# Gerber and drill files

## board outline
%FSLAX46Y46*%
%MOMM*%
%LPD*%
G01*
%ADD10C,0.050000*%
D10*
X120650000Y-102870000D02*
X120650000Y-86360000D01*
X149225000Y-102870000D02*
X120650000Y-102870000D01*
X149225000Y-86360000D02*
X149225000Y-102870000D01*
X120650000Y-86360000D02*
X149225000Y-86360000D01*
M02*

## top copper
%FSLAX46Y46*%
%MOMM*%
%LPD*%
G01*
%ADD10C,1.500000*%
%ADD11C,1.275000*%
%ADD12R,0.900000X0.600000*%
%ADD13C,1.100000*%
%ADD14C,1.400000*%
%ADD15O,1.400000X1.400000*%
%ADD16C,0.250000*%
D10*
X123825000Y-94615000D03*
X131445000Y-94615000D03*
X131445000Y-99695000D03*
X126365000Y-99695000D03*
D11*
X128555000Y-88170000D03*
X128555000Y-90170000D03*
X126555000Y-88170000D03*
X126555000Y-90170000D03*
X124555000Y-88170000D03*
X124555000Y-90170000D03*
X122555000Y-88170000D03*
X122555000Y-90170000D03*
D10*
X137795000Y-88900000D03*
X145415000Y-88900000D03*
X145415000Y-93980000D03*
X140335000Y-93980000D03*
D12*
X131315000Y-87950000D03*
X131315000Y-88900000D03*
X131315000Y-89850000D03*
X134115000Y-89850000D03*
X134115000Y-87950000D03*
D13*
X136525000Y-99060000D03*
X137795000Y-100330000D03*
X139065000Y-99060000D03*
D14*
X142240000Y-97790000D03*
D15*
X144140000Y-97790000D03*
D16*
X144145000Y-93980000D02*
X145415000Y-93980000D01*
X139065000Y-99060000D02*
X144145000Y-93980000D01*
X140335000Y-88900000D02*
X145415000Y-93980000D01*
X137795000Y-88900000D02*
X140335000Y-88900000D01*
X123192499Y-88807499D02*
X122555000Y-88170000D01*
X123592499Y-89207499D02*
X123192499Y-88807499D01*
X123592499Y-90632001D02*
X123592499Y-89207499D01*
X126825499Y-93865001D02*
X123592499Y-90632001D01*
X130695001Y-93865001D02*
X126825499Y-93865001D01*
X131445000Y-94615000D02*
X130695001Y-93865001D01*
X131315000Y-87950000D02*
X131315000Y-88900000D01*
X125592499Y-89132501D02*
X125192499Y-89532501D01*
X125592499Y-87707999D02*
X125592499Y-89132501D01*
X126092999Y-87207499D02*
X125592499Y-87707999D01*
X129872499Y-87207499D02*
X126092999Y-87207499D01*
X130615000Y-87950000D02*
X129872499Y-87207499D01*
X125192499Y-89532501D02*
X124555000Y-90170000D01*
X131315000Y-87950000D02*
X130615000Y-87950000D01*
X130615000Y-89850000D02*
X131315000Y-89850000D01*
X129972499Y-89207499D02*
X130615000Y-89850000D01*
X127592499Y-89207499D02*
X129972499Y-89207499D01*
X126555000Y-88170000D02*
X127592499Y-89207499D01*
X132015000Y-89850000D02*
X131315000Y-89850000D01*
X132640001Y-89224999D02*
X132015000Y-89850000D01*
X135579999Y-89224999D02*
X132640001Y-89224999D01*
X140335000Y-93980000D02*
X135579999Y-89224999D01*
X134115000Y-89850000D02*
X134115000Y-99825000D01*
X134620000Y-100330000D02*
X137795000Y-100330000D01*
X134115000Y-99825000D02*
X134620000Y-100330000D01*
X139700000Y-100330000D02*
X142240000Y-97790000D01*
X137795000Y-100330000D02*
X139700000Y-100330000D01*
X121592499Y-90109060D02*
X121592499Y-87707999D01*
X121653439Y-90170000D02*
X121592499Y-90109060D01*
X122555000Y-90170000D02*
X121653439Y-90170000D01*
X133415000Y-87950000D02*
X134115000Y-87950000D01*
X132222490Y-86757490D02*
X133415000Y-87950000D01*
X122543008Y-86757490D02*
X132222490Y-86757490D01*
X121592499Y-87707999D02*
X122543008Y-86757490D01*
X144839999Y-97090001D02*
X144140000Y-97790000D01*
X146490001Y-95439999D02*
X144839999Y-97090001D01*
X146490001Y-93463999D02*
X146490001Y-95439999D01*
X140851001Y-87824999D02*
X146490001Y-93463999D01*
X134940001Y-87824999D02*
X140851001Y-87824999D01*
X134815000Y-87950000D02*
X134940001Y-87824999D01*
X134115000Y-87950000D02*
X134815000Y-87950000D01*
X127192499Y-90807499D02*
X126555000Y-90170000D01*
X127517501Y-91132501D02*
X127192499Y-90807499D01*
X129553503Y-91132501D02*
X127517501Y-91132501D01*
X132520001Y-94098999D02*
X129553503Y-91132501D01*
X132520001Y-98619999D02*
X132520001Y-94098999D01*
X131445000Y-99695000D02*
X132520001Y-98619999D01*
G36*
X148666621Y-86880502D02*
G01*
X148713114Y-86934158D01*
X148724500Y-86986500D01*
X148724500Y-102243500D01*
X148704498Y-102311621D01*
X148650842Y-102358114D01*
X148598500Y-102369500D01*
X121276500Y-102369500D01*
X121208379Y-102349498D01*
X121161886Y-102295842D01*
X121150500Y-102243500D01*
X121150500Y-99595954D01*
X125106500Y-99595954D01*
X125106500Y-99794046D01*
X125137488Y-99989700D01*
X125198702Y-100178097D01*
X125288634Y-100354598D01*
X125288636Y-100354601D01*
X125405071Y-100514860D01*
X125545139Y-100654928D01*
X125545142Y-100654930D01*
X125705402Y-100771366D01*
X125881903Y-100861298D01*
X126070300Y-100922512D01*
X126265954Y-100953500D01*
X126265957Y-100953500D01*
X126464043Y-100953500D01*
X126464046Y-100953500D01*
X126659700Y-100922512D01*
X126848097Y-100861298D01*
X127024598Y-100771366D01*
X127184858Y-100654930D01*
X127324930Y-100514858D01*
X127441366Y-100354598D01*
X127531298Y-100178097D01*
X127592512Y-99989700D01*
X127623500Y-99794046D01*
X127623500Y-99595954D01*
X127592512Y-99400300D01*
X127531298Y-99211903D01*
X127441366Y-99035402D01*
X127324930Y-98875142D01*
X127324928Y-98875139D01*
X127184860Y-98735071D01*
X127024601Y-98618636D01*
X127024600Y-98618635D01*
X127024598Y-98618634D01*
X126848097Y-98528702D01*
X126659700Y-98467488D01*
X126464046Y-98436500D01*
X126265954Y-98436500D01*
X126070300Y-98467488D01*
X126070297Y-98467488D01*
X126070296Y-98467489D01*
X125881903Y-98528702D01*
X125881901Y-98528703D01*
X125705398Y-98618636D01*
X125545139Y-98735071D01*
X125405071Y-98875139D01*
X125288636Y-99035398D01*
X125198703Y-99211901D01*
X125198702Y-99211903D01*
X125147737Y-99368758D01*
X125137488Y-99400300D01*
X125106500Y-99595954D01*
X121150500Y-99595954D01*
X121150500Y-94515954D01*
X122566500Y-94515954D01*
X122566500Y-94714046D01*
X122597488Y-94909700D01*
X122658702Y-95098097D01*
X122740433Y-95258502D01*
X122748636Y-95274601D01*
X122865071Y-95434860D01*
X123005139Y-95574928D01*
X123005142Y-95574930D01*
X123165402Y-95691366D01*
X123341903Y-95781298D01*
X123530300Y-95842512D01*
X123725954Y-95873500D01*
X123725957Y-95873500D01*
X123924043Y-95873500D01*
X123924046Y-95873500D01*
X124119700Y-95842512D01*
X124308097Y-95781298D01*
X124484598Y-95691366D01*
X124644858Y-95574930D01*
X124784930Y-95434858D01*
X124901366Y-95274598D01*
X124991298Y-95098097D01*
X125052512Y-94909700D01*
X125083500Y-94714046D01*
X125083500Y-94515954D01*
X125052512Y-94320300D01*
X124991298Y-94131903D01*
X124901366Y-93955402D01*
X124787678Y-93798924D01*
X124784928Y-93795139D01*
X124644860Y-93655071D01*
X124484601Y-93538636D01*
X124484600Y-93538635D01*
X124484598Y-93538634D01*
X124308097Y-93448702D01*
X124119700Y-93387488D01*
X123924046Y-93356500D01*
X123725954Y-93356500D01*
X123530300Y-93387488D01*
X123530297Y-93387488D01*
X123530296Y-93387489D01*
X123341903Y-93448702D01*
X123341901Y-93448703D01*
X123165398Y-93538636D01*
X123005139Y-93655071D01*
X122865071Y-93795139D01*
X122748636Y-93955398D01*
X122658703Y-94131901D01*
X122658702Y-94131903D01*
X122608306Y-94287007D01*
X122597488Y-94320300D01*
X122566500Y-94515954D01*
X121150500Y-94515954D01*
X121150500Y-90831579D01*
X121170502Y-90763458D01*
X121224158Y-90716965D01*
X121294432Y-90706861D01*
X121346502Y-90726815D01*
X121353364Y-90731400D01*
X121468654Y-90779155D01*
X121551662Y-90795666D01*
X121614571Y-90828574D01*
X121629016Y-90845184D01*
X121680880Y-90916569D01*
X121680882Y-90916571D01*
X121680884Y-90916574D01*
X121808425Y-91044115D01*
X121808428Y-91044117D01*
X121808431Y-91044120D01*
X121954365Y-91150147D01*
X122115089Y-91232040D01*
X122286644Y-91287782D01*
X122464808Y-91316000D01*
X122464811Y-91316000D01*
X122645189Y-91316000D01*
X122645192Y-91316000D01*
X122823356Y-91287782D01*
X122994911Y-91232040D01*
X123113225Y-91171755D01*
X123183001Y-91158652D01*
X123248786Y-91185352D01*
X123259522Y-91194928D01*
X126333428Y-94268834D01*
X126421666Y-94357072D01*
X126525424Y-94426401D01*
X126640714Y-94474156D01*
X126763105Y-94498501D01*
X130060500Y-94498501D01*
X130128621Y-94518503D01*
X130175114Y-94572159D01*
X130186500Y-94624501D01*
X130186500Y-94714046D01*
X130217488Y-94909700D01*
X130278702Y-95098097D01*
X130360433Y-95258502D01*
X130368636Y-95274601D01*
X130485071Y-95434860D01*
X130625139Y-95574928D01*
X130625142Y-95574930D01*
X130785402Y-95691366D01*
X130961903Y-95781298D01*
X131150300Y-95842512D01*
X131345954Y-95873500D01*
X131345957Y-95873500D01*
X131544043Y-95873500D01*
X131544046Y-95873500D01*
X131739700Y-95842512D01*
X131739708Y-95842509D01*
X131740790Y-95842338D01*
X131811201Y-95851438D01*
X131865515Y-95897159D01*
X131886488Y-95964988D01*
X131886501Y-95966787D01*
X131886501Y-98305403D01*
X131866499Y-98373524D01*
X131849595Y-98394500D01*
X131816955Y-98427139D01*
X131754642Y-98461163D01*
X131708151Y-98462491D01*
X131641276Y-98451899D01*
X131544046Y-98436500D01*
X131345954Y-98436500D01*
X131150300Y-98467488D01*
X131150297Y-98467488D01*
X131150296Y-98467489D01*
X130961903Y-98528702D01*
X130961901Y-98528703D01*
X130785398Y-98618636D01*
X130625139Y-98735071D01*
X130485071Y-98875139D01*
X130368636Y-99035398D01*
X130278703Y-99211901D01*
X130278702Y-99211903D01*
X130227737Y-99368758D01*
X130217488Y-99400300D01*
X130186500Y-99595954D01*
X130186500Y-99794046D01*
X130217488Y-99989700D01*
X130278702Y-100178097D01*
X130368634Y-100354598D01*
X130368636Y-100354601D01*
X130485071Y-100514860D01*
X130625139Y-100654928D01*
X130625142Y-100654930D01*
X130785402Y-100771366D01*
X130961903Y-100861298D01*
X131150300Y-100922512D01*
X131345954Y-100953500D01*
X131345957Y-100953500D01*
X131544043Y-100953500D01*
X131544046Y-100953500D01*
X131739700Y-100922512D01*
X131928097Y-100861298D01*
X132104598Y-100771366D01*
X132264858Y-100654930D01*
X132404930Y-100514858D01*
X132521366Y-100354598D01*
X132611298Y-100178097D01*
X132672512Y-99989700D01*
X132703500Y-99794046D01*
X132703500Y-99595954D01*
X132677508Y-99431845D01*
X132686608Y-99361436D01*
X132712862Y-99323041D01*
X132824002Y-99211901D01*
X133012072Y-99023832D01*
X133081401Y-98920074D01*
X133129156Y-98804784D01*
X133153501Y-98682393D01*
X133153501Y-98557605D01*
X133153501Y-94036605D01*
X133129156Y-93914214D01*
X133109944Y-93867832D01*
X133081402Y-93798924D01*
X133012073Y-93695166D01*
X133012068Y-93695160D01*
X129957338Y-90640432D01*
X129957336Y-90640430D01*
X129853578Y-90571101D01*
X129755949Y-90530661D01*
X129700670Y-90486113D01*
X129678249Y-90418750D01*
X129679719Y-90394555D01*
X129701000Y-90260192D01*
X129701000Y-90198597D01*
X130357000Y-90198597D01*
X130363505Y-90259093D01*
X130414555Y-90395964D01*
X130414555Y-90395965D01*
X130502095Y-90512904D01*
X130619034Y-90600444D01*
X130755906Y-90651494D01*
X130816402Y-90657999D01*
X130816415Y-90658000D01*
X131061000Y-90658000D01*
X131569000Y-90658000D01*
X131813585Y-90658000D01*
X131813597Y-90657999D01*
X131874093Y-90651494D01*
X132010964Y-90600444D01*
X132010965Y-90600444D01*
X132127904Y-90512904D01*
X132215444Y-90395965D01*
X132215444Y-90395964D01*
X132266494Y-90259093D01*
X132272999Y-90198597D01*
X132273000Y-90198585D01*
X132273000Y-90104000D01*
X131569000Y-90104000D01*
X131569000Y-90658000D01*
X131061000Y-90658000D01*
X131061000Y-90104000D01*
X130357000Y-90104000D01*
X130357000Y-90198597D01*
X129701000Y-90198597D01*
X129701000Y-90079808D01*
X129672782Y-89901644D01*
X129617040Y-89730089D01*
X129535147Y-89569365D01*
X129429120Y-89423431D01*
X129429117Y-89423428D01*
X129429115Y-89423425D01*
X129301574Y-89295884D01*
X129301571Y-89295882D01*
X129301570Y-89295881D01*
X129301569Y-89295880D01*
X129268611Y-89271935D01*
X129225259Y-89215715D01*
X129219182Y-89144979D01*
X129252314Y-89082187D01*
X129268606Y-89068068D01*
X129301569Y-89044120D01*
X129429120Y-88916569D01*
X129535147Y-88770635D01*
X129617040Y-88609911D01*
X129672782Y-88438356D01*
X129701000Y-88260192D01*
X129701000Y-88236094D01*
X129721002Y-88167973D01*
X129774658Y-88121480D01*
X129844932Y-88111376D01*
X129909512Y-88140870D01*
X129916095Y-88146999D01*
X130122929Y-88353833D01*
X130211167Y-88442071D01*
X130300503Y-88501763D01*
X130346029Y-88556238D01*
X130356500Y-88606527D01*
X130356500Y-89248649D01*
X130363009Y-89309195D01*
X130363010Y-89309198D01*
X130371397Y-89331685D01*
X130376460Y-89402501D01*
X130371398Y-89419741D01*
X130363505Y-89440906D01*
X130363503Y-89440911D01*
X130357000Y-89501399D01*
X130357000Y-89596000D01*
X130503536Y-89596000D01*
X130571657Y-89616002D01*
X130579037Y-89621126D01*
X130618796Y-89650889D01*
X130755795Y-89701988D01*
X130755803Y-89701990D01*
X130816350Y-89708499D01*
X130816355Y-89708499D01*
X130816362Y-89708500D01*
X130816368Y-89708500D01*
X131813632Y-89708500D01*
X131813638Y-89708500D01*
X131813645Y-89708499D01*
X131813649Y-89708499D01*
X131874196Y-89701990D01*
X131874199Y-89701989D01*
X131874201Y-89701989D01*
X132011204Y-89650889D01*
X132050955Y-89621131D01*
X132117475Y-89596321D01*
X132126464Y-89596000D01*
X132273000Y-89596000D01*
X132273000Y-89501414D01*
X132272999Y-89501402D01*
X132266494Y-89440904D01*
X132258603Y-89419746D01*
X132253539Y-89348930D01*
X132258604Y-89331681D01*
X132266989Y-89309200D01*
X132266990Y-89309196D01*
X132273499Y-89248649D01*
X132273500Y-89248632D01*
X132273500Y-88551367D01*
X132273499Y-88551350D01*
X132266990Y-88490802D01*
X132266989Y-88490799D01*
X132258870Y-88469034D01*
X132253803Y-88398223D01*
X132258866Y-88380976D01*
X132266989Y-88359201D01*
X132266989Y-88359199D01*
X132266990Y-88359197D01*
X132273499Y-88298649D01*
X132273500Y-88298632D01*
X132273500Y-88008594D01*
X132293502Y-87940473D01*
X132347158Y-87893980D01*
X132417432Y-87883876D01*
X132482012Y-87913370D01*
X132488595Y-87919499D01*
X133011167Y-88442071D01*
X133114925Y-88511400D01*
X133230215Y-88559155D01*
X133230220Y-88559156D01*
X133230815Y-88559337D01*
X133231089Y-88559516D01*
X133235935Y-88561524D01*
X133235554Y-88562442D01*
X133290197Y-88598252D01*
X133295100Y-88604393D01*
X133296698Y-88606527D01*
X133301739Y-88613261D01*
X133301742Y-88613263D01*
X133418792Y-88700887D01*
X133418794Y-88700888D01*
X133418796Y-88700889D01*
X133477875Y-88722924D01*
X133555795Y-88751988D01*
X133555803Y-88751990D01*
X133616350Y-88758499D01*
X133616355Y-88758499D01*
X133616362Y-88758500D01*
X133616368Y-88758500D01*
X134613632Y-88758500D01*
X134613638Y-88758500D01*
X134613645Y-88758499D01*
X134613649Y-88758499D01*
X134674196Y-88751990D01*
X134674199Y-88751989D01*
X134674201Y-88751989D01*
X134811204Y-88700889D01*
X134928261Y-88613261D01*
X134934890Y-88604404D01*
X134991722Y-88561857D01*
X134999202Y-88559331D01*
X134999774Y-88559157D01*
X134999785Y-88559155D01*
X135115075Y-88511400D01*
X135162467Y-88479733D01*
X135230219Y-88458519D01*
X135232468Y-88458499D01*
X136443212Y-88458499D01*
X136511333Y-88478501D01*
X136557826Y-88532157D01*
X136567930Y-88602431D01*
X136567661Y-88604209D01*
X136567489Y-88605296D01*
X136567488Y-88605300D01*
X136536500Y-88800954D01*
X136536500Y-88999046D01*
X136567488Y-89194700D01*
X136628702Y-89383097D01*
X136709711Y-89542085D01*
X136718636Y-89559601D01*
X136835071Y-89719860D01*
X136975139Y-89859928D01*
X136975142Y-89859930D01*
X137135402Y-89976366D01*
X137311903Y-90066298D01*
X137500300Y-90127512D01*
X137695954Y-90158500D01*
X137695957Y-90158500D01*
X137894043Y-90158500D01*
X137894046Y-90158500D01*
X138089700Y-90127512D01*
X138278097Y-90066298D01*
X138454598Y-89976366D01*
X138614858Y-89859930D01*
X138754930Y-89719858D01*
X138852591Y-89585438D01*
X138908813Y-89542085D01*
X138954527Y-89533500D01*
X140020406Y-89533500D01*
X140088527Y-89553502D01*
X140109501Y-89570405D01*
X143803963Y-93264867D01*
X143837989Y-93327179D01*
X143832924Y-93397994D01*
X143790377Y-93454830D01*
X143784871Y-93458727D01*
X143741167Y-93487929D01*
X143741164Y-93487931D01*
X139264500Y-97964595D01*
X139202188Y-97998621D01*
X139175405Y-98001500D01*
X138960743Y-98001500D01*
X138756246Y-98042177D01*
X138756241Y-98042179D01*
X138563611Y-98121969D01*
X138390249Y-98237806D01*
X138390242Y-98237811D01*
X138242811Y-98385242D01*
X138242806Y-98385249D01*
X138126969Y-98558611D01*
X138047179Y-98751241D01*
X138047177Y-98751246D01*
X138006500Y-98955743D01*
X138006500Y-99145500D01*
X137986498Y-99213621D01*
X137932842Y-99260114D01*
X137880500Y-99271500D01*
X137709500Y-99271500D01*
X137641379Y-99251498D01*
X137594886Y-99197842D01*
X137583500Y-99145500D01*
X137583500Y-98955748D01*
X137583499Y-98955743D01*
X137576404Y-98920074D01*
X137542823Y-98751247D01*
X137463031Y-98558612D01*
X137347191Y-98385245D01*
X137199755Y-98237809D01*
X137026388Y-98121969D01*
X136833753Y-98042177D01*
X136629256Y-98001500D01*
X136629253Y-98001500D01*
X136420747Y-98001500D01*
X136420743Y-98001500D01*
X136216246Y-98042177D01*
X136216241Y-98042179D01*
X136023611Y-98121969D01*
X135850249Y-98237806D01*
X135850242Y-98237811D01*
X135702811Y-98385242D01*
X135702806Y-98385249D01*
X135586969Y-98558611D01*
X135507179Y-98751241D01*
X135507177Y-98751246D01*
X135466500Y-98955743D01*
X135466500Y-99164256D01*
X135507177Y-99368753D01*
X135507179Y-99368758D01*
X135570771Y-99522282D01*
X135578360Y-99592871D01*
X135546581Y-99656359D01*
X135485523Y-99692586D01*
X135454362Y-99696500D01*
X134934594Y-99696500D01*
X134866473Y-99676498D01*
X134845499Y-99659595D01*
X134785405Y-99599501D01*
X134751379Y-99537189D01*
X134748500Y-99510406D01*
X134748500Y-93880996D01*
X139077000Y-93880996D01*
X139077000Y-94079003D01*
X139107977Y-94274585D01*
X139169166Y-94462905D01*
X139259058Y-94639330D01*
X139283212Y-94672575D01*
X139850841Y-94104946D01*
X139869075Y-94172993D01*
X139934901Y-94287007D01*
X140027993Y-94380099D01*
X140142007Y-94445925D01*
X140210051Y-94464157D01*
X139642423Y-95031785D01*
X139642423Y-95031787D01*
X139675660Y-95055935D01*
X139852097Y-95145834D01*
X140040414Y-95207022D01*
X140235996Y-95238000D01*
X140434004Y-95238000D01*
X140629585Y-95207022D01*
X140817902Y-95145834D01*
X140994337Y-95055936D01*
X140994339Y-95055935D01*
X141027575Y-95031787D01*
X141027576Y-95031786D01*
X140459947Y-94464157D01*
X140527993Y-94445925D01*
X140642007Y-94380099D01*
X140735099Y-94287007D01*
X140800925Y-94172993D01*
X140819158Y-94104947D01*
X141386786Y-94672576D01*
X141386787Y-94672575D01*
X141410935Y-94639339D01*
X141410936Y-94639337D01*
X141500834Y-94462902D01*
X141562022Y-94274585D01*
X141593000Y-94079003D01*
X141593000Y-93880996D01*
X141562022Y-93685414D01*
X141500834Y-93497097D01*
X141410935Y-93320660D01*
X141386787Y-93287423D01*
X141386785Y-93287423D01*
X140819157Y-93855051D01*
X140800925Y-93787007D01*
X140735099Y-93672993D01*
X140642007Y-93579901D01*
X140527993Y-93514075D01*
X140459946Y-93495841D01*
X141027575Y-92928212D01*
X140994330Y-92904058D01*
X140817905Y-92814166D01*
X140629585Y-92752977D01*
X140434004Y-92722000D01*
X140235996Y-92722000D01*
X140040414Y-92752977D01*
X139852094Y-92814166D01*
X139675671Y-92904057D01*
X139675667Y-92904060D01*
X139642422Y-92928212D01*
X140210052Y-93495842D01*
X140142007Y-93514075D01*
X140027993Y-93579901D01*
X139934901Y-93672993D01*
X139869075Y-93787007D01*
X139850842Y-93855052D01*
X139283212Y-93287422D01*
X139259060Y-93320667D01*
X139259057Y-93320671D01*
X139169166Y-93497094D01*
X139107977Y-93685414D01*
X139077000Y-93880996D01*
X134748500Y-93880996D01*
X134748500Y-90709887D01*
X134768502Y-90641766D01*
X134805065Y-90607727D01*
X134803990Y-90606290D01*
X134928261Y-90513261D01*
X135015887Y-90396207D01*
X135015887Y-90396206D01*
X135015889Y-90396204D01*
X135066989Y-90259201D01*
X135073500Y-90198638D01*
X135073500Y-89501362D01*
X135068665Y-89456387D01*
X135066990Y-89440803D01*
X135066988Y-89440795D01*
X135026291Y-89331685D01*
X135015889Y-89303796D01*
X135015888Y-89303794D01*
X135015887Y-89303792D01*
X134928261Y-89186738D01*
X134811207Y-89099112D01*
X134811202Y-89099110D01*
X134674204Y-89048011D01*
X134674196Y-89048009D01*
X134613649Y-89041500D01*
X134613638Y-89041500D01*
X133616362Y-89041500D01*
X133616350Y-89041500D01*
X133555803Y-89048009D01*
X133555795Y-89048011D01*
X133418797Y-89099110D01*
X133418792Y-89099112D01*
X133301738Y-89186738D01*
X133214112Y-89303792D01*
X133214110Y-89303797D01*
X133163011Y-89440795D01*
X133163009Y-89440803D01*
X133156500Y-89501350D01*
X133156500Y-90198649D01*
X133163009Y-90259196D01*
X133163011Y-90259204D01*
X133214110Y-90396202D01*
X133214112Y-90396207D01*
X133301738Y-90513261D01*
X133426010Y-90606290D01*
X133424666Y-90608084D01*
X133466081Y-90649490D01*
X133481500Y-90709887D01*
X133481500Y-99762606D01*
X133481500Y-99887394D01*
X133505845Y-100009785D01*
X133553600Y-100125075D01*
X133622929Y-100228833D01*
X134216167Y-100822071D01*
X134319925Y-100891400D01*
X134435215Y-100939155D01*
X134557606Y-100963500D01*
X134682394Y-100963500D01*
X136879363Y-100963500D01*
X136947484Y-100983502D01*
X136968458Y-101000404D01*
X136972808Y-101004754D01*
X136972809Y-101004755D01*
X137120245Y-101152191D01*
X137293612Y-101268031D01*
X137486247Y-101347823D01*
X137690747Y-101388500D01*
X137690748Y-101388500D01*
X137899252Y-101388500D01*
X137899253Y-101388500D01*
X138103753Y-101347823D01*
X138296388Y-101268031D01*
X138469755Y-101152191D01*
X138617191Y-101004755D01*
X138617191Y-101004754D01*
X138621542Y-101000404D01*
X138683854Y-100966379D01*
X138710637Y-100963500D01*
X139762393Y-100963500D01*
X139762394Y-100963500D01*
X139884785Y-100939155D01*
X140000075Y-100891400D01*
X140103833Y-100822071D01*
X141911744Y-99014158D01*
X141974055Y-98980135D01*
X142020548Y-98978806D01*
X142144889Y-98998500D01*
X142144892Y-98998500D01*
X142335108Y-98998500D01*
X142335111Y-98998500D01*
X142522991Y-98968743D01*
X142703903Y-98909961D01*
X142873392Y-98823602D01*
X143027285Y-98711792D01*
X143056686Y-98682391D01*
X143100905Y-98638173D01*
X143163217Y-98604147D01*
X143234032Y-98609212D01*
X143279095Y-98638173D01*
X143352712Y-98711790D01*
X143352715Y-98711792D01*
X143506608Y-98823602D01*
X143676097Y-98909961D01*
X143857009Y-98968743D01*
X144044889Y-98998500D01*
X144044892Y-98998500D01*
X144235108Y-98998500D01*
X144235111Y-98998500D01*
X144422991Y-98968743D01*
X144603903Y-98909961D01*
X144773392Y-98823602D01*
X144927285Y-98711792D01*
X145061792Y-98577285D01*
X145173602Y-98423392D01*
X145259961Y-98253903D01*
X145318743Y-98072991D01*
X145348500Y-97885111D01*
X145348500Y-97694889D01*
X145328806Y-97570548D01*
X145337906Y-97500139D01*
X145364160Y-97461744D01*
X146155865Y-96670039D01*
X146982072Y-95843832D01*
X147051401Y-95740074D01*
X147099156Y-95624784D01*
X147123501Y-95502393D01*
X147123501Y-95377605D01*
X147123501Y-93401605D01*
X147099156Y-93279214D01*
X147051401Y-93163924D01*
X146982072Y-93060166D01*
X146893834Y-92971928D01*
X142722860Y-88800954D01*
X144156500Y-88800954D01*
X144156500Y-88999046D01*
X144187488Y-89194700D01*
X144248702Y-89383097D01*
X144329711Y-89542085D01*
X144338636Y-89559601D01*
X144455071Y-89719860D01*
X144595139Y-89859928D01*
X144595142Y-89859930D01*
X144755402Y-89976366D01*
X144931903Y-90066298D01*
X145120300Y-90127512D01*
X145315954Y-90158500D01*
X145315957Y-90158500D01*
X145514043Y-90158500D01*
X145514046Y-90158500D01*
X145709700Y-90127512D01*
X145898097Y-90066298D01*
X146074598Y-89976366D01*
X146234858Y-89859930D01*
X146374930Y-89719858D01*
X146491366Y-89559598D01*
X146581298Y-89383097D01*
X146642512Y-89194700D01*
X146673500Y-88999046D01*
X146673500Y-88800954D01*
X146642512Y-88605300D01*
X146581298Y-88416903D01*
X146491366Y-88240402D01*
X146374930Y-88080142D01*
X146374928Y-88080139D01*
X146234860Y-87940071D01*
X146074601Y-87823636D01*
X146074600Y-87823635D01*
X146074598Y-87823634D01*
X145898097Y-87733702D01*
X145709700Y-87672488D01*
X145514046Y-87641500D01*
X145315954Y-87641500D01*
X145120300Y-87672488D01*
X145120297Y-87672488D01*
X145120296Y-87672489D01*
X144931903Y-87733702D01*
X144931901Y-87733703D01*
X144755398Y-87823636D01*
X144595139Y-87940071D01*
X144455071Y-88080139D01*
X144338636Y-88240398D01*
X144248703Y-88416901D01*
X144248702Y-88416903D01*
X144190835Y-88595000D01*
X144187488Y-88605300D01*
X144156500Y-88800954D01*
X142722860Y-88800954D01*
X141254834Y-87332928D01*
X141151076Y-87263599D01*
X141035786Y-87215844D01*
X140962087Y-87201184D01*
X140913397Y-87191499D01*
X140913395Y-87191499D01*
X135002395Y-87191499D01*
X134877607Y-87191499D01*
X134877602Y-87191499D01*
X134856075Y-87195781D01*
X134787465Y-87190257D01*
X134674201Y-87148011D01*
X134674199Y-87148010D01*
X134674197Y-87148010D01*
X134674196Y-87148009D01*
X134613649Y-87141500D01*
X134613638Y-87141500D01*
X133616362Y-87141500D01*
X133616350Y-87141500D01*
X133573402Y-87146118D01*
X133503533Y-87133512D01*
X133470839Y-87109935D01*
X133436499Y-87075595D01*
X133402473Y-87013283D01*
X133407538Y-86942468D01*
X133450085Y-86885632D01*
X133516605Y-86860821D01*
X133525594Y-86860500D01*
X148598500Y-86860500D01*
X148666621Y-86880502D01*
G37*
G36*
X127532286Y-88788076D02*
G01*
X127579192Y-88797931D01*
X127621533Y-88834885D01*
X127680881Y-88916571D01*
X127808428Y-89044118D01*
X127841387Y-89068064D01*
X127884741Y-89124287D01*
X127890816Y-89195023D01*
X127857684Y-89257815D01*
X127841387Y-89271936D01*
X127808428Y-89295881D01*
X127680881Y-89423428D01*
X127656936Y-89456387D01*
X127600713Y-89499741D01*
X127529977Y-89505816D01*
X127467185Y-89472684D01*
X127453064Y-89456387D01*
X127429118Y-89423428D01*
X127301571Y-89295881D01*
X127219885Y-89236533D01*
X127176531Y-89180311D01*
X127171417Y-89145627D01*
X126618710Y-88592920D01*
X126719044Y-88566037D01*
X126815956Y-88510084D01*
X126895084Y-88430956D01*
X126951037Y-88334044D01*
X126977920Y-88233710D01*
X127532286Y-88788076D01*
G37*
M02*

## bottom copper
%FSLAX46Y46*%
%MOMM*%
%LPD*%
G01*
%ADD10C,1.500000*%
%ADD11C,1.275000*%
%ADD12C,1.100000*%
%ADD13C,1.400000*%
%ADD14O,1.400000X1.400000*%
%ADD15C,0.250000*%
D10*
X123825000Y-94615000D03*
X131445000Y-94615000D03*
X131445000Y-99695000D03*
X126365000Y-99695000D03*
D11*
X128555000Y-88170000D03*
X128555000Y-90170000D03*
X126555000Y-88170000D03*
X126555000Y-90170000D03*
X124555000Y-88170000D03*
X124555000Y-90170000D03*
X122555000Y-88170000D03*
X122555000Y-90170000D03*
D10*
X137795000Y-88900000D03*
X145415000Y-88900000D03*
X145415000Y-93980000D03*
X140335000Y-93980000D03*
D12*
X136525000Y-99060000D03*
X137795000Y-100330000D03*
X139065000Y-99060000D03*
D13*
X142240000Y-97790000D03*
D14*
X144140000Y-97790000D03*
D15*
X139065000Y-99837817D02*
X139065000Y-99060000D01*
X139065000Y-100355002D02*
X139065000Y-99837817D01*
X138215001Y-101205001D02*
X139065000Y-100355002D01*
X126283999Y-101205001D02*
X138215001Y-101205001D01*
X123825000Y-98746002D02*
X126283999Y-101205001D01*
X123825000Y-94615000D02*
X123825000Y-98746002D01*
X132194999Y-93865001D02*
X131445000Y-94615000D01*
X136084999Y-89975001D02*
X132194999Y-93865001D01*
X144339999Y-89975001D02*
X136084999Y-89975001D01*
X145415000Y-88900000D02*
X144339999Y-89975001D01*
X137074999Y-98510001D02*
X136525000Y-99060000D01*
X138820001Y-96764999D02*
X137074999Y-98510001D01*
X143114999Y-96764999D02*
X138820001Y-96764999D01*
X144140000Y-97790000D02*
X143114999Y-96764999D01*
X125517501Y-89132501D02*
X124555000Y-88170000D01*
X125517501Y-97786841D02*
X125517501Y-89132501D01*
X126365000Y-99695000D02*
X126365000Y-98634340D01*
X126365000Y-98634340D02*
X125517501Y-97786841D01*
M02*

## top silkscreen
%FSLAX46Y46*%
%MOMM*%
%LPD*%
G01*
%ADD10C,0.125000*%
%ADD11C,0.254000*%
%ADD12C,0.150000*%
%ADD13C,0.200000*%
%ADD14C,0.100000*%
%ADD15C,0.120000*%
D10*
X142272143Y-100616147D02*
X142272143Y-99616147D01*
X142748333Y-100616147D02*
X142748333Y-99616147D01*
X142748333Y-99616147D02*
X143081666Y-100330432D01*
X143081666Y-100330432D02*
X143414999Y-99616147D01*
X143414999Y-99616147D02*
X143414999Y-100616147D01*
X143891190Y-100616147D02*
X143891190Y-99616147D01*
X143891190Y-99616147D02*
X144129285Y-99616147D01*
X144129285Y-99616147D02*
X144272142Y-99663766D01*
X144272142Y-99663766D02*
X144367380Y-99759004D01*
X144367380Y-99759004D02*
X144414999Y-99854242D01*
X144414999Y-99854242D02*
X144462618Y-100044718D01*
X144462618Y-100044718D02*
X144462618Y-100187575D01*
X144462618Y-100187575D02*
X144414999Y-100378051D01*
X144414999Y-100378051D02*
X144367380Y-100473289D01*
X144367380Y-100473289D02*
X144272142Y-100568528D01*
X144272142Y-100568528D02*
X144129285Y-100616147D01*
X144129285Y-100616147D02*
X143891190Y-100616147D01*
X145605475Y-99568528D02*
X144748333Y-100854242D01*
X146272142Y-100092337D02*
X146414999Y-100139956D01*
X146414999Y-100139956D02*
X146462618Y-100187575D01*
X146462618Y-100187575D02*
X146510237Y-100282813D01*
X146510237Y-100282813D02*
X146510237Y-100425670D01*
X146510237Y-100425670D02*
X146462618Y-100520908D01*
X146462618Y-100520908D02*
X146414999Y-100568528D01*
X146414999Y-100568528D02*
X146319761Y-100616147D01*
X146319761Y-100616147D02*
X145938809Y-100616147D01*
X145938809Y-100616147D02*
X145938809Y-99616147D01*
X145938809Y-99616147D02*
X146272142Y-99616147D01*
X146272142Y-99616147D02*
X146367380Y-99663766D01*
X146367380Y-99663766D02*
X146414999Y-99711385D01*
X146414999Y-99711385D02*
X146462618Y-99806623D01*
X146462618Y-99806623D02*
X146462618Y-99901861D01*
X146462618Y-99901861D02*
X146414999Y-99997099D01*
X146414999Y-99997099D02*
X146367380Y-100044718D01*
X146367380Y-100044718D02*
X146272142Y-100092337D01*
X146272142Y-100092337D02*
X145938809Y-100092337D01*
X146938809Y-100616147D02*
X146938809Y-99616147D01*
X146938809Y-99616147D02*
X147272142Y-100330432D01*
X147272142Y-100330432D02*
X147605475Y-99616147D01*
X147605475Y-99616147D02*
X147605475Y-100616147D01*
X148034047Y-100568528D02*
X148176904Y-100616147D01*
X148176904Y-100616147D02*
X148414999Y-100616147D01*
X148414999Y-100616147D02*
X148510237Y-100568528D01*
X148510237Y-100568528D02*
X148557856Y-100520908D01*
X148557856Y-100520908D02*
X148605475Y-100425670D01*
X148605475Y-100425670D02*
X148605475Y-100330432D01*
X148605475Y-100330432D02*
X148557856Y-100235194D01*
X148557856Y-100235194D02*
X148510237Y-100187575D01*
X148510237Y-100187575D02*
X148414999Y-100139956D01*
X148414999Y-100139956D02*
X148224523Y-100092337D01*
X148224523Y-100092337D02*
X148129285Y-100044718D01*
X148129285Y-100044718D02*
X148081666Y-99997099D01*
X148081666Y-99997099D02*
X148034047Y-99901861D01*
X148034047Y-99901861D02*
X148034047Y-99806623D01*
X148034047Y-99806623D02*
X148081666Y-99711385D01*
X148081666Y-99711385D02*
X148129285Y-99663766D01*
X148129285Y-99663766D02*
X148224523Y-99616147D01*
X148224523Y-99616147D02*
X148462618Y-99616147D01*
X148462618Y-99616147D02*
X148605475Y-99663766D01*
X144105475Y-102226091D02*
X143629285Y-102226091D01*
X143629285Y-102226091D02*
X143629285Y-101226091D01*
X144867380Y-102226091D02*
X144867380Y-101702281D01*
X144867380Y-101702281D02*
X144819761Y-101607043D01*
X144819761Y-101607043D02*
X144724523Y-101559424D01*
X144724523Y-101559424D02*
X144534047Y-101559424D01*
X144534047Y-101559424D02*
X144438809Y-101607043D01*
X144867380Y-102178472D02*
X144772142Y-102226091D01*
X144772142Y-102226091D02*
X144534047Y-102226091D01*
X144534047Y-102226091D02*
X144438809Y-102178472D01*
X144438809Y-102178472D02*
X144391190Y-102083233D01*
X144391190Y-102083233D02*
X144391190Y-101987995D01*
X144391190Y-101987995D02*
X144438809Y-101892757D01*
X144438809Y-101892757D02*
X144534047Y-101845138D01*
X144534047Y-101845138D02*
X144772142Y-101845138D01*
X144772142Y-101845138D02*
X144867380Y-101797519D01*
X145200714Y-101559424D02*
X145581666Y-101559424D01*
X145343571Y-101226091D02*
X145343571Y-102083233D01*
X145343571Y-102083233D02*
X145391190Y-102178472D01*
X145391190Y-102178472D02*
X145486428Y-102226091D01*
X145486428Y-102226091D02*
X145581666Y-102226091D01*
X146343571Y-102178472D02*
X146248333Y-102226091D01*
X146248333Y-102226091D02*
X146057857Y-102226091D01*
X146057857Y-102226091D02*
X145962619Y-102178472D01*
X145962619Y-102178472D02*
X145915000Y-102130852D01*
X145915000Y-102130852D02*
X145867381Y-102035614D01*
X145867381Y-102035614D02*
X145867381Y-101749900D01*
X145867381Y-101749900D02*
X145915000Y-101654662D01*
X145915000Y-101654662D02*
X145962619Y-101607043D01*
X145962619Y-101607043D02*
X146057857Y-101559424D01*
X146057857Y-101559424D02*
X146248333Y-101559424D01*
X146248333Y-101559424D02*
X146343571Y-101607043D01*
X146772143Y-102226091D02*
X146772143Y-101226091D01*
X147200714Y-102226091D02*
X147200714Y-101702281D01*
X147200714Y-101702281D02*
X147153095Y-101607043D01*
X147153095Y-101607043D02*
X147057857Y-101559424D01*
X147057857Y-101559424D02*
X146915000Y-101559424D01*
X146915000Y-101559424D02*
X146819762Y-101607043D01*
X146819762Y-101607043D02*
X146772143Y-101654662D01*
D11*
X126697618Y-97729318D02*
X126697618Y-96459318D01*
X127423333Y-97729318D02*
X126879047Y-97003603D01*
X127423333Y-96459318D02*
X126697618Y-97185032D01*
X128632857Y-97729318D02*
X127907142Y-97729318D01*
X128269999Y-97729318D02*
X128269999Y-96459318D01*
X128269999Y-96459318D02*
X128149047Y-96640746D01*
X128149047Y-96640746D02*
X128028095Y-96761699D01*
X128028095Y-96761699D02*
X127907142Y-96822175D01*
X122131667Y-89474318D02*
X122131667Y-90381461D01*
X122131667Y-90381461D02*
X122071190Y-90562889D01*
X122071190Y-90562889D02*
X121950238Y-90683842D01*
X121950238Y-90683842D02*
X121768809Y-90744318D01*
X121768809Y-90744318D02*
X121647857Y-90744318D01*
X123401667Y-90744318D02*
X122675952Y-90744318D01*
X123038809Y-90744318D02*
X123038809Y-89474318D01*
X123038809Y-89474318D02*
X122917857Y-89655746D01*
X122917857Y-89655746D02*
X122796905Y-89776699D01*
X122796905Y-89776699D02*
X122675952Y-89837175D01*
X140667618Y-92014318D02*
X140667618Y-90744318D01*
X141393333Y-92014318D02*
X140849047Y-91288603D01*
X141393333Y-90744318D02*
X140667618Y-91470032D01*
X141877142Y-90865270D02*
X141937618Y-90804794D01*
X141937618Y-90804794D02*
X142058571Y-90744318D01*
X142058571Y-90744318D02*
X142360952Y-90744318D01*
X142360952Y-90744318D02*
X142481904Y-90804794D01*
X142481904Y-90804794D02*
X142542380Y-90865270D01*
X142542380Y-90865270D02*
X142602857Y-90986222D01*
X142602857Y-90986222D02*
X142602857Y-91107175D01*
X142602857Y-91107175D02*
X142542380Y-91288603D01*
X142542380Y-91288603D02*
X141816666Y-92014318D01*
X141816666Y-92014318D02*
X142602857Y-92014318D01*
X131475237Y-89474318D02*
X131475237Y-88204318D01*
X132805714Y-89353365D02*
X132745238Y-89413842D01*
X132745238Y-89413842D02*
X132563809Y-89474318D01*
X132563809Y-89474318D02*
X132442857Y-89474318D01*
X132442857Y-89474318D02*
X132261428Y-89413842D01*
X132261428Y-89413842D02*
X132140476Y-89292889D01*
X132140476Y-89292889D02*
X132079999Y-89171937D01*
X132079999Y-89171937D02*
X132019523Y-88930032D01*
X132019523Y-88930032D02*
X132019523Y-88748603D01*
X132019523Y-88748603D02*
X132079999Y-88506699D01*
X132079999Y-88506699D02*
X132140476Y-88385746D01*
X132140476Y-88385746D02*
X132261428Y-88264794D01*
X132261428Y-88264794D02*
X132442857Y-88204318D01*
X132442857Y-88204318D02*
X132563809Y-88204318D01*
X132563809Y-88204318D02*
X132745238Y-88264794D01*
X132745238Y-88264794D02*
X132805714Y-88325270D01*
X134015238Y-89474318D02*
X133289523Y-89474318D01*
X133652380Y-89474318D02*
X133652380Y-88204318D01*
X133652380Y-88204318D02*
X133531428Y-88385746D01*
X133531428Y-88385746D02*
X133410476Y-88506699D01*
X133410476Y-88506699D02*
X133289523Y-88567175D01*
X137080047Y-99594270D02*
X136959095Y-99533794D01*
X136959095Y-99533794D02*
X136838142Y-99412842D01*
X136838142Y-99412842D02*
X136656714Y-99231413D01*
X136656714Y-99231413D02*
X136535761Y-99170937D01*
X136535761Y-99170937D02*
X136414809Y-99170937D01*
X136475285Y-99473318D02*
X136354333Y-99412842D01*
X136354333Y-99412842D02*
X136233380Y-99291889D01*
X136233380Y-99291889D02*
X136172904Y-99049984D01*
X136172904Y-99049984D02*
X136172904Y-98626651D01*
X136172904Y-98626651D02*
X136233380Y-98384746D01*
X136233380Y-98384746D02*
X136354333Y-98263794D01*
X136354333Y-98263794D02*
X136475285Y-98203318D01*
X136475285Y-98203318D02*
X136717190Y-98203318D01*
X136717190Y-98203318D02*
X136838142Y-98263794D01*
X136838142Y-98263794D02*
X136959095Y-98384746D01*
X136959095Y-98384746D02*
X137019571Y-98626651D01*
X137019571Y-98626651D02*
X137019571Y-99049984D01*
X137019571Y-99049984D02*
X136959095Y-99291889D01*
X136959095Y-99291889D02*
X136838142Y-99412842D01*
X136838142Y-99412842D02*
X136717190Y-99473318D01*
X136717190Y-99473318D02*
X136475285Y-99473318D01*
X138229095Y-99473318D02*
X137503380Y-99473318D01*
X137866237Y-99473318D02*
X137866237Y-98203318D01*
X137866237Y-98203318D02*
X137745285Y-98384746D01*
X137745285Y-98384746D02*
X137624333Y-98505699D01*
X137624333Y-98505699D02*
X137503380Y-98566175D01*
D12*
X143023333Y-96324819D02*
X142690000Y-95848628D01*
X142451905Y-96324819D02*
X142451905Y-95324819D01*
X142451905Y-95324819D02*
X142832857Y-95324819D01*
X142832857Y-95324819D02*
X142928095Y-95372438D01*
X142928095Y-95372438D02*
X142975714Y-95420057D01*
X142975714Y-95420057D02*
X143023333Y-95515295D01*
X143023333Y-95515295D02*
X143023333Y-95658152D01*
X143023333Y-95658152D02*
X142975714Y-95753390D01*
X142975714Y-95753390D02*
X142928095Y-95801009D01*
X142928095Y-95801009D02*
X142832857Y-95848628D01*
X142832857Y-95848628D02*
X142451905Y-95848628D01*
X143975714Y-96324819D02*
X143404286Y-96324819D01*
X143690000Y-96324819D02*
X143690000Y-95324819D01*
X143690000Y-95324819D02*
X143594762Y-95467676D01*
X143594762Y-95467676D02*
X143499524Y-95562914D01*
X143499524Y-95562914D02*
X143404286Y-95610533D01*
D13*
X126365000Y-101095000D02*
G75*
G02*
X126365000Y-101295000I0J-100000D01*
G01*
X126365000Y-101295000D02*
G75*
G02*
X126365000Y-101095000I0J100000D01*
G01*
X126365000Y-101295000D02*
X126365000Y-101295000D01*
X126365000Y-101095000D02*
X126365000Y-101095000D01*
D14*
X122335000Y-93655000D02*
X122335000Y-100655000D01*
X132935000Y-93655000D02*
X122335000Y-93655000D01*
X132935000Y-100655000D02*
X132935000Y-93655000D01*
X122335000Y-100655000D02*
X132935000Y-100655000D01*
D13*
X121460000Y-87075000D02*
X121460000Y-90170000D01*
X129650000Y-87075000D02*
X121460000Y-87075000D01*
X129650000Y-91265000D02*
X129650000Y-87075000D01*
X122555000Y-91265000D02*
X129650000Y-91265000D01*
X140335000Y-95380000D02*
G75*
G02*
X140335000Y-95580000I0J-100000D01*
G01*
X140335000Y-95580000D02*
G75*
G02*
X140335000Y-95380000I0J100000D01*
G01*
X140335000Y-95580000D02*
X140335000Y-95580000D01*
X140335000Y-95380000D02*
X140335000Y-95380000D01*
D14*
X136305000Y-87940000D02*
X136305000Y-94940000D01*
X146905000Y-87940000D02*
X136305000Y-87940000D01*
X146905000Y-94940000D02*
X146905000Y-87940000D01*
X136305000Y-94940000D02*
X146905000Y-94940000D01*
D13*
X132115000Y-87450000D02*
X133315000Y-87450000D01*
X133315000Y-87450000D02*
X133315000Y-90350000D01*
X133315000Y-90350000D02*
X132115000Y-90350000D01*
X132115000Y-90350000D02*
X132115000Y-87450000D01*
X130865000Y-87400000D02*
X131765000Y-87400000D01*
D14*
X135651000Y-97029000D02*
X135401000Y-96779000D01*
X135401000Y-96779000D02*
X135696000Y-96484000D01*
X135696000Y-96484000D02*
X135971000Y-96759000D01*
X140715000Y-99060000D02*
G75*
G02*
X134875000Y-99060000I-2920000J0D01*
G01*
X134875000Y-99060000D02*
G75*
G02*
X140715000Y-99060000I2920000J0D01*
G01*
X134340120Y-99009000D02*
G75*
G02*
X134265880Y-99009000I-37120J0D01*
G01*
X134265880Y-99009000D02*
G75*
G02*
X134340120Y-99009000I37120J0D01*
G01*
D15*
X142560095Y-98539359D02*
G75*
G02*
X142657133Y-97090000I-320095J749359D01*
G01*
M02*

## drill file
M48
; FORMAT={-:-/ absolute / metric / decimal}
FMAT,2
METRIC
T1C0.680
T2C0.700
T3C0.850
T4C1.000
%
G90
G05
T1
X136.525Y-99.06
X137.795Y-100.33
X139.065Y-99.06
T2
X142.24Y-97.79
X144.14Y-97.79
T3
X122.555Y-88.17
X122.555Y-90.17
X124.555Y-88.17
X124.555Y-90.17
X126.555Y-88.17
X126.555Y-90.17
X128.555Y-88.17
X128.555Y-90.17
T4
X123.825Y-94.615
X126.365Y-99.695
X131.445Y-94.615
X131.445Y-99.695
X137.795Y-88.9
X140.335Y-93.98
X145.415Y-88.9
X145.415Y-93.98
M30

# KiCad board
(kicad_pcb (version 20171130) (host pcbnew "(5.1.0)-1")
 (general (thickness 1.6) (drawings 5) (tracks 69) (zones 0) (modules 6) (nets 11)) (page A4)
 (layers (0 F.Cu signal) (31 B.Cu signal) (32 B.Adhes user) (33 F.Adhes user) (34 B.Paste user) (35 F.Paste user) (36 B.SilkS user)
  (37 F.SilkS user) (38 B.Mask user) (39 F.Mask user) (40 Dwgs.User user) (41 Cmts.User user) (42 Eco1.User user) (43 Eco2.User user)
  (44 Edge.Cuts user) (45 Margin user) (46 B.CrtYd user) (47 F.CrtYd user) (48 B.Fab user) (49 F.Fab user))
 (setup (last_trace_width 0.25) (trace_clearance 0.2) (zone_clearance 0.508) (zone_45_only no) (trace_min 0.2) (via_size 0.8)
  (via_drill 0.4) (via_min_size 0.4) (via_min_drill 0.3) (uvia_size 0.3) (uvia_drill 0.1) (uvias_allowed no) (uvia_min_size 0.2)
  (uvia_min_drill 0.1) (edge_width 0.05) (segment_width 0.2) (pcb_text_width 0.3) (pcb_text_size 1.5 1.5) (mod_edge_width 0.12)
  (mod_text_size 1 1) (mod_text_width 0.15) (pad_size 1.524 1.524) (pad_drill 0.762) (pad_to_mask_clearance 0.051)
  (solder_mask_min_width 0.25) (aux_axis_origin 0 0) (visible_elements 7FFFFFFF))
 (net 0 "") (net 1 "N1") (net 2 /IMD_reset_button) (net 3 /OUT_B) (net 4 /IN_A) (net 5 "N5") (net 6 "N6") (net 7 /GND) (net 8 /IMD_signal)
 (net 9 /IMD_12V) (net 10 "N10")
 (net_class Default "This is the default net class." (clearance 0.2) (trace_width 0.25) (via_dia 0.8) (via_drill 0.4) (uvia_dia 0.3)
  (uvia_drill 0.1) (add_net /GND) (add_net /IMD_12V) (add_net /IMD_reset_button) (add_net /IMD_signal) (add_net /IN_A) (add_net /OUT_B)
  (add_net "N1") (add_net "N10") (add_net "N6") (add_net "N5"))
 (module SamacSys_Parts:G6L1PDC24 (layer F.Cu) (at 126.365 99.695)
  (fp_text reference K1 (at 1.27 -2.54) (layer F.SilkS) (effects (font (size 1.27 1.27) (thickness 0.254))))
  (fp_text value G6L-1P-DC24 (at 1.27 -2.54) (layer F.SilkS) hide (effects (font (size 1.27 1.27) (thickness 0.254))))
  (fp_arc (start 0 1.5) (end 0 1.6) (angle -180) (layer F.SilkS) (width 0.2))
  (fp_arc (start 0 1.5) (end 0 1.4) (angle -180) (layer F.SilkS) (width 0.2))
  (fp_line (start 0 1.6) (end 0 1.6) (layer F.SilkS) (width 0.2))
  (fp_line (start 0 1.4) (end 0 1.4) (layer F.SilkS) (width 0.2))
  (fp_line (start -4.03 -6.04) (end -4.03 0.96) (layer F.SilkS) (width 0.1))
  (fp_line (start 6.57 -6.04) (end -4.03 -6.04) (layer F.SilkS) (width 0.1))
  (fp_line (start 6.57 0.96) (end 6.57 -6.04) (layer F.SilkS) (width 0.1))
  (fp_line (start -4.03 0.96) (end 6.57 0.96) (layer F.SilkS) (width 0.1))
  (pad 8 thru_hole circle (at -2.54 -5.08) (size 1.5 1.5) (drill 1) (layers *.Cu *.Mask) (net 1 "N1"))
  (pad 5 thru_hole circle (at 5.08 -5.08) (size 1.5 1.5) (drill 1) (layers *.Cu *.Mask) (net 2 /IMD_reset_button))
  (pad 4 thru_hole circle (at 5.08 0) (size 1.5 1.5) (drill 1) (layers *.Cu *.Mask) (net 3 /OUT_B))
  (pad 2 thru_hole circle (at 0 0) (size 1.5 1.5) (drill 1) (layers *.Cu *.Mask) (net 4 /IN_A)))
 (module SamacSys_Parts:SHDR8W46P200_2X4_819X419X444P (layer F.Cu) (at 122.555 90.17)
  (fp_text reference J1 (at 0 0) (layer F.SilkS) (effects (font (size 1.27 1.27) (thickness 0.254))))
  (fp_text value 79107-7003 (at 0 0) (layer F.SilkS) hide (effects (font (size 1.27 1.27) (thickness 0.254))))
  (fp_line (start -1.095 -3.095) (end -1.095 0) (layer F.SilkS) (width 0.2))
  (fp_line (start 7.095 -3.095) (end -1.095 -3.095) (layer F.SilkS) (width 0.2))
  (fp_line (start 7.095 1.095) (end 7.095 -3.095) (layer F.SilkS) (width 0.2))
  (fp_line (start 0 1.095) (end 7.095 1.095) (layer F.SilkS) (width 0.2))
  (pad 8 thru_hole circle (at 6 -2) (size 1.275 1.275) (drill 0.85) (layers *.Cu *.Mask) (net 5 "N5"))
  (pad 7 thru_hole circle (at 6 0) (size 1.275 1.275) (drill 0.85) (layers *.Cu *.Mask) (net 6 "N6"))
  (pad 6 thru_hole circle (at 4 -2) (size 1.275 1.275) (drill 0.85) (layers *.Cu *.Mask) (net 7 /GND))
  (pad 5 thru_hole circle (at 4 0) (size 1.275 1.275) (drill 0.85) (layers *.Cu *.Mask) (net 3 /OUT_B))
  (pad 4 thru_hole circle (at 2 -2) (size 1.275 1.275) (drill 0.85) (layers *.Cu *.Mask) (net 4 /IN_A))
  (pad 3 thru_hole circle (at 2 0) (size 1.275 1.275) (drill 0.85) (layers *.Cu *.Mask) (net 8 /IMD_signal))
  (pad 2 thru_hole circle (at 0 -2) (size 1.275 1.275) (drill 0.85) (layers *.Cu *.Mask) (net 2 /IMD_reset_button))
  (pad 1 thru_hole circle (at 0 0) (size 1.275 1.275) (drill 0.85) (layers *.Cu *.Mask) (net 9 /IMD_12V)))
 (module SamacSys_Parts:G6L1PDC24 (layer F.Cu) (at 140.335 93.98)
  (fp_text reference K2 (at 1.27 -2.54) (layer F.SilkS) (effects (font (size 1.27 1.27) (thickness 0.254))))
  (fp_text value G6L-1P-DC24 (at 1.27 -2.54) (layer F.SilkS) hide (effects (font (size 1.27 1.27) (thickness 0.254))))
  (fp_arc (start 0 1.5) (end 0 1.6) (angle -180) (layer F.SilkS) (width 0.2))
  (fp_arc (start 0 1.5) (end 0 1.4) (angle -180) (layer F.SilkS) (width 0.2))
  (fp_line (start 0 1.6) (end 0 1.6) (layer F.SilkS) (width 0.2))
  (fp_line (start 0 1.4) (end 0 1.4) (layer F.SilkS) (width 0.2))
  (fp_line (start -4.03 -6.04) (end -4.03 0.96) (layer F.SilkS) (width 0.1))
  (fp_line (start 6.57 -6.04) (end -4.03 -6.04) (layer F.SilkS) (width 0.1))
  (fp_line (start 6.57 0.96) (end 6.57 -6.04) (layer F.SilkS) (width 0.1))
  (fp_line (start -4.03 0.96) (end 6.57 0.96) (layer F.SilkS) (width 0.1))
  (pad 8 thru_hole circle (at -2.54 -5.08) (size 1.5 1.5) (drill 1) (layers *.Cu *.Mask) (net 1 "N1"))
  (pad 5 thru_hole circle (at 5.08 -5.08) (size 1.5 1.5) (drill 1) (layers *.Cu *.Mask) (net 2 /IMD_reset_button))
  (pad 4 thru_hole circle (at 5.08 0) (size 1.5 1.5) (drill 1) (layers *.Cu *.Mask) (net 1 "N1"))
  (pad 2 thru_hole circle (at 0 0) (size 1.5 1.5) (drill 1) (layers *.Cu *.Mask) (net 7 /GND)))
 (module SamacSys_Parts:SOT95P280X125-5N (layer F.Cu) (at 132.715 88.9)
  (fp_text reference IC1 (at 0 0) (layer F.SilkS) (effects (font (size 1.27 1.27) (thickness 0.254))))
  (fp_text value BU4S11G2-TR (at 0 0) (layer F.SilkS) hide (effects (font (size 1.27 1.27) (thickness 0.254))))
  (fp_line (start -0.6 -1.45) (end 0.6 -1.45) (layer F.SilkS) (width 0.2))
  (fp_line (start 0.6 -1.45) (end 0.6 1.45) (layer F.SilkS) (width 0.2))
  (fp_line (start 0.6 1.45) (end -0.6 1.45) (layer F.SilkS) (width 0.2))
  (fp_line (start -0.6 1.45) (end -0.6 -1.45) (layer F.SilkS) (width 0.2))
  (fp_line (start -1.85 -1.5) (end -0.95 -1.5) (layer F.SilkS) (width 0.2))
  (pad 1 smd rect (at -1.4 -0.95 90) (size 0.6 0.9) (layers F.Cu F.Paste F.Mask) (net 8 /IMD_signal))
  (pad 2 smd rect (at -1.4 0 90) (size 0.6 0.9) (layers F.Cu F.Paste F.Mask) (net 8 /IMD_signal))
  (pad 3 smd rect (at -1.4 0.95 90) (size 0.6 0.9) (layers F.Cu F.Paste F.Mask) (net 7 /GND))
  (pad 4 smd rect (at 1.4 0.95 90) (size 0.6 0.9) (layers F.Cu F.Paste F.Mask) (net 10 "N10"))
  (pad 5 smd rect (at 1.4 -0.95 90) (size 0.6 0.9) (layers F.Cu F.Paste F.Mask) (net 9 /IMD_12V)))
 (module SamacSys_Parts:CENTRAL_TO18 (layer F.Cu) (at 137.795 99.06)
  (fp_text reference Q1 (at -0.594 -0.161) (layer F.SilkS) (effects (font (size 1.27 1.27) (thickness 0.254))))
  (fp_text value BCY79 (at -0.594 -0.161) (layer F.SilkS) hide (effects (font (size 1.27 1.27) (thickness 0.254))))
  (fp_line (start -2.144 -2.031) (end -2.394 -2.281) (layer F.SilkS) (width 0.1))
  (fp_line (start -2.394 -2.281) (end -2.099 -2.576) (layer F.SilkS) (width 0.1))
  (fp_line (start -2.099 -2.576) (end -1.824 -2.301) (layer F.SilkS) (width 0.1))
  (fp_circle (center 0 0) (end 0 2.92) (layer F.SilkS) (width 0.1))
  (fp_circle (center -3.492 -0.051) (end -3.492 -0.01388) (layer F.SilkS) (width 0.1))
  (pad 1 thru_hole circle (at -1.27 0) (size 1.1 1.1) (drill 0.68) (layers *.Cu *.Mask) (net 9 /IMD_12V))
  (pad 2 thru_hole circle (at 0 1.27) (size 1.1 1.1) (drill 0.68) (layers *.Cu *.Mask) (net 10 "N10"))
  (pad 3 thru_hole circle (at 1.27 0) (size 1.1 1.1) (drill 0.68) (layers *.Cu *.Mask) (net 1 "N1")))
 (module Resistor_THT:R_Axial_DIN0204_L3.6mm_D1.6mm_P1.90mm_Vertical (layer F.Cu) (at 142.24 97.79)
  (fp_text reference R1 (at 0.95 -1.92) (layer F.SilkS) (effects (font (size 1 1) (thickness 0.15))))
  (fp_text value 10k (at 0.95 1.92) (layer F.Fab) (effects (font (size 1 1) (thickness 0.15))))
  (fp_arc (start 0 0) (end 0.417133 -0.7) (angle -233.92106) (layer F.SilkS) (width 0.12))
  (pad 1 thru_hole circle (at 0 0) (size 1.4 1.4) (drill 0.7) (layers *.Cu *.Mask) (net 10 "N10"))
  (pad 2 thru_hole oval (at 1.9 0) (size 1.4 1.4) (drill 0.7) (layers *.Cu *.Mask) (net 9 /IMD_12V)))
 (gr_line (start 120.65 102.87) (end 120.65 86.36) (layer Edge.Cuts) (width 0.05))
 (gr_line (start 149.225 102.87) (end 120.65 102.87) (layer Edge.Cuts) (width 0.05))
 (gr_line (start 149.225 86.36) (end 149.225 102.87) (layer Edge.Cuts) (width 0.05))
 (gr_line (start 120.65 86.36) (end 149.225 86.36) (layer Edge.Cuts) (width 0.05))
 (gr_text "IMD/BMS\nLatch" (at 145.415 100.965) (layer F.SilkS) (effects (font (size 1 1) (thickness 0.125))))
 (segment (start 144.145 93.98) (end 145.415 93.98) (width 0.25) (layer F.Cu) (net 1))
 (segment (start 139.065 99.06) (end 144.145 93.98) (width 0.25) (layer F.Cu) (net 1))
 (segment (start 140.335 88.9) (end 145.415 93.98) (width 0.25) (layer F.Cu) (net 1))
 (segment (start 137.795 88.9) (end 140.335 88.9) (width 0.25) (layer F.Cu) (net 1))
 (segment (start 139.065 99.837817) (end 139.065 99.06) (width 0.25) (layer B.Cu) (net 1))
 (segment (start 139.065 100.355002) (end 139.065 99.837817) (width 0.25) (layer B.Cu) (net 1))
 (segment (start 138.215001 101.205001) (end 139.065 100.355002) (width 0.25) (layer B.Cu) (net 1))
 (segment (start 126.283999 101.205001) (end 138.215001 101.205001) (width 0.25) (layer B.Cu) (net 1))
 (segment (start 123.825 98.746002) (end 126.283999 101.205001) (width 0.25) (layer B.Cu) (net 1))
 (segment (start 123.825 94.615) (end 123.825 98.746002) (width 0.25) (layer B.Cu) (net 1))
 (segment (start 123.192499 88.807499) (end 122.555 88.17) (width 0.25) (layer F.Cu) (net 2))
 (segment (start 123.592499 89.207499) (end 123.192499 88.807499) (width 0.25) (layer F.Cu) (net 2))
 (segment (start 123.592499 90.632001) (end 123.592499 89.207499) (width 0.25) (layer F.Cu) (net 2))
 (segment (start 126.825499 93.865001) (end 123.592499 90.632001) (width 0.25) (layer F.Cu) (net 2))
 (segment (start 130.695001 93.865001) (end 126.825499 93.865001) (width 0.25) (layer F.Cu) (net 2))
 (segment (start 131.445 94.615) (end 130.695001 93.865001) (width 0.25) (layer F.Cu) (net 2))
 (segment (start 132.194999 93.865001) (end 131.445 94.615) (width 0.25) (layer B.Cu) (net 2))
 (segment (start 136.084999 89.975001) (end 132.194999 93.865001) (width 0.25) (layer B.Cu) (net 2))
 (segment (start 144.339999 89.975001) (end 136.084999 89.975001) (width 0.25) (layer B.Cu) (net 2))
 (segment (start 145.415 88.9) (end 144.339999 89.975001) (width 0.25) (layer B.Cu) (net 2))
 (segment (start 131.315 87.95) (end 131.315 88.9) (width 0.25) (layer F.Cu) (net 8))
 (segment (start 125.592499 89.132501) (end 125.192499 89.532501) (width 0.25) (layer F.Cu) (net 8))
 (segment (start 125.592499 87.707999) (end 125.592499 89.132501) (width 0.25) (layer F.Cu) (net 8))
 (segment (start 126.092999 87.207499) (end 125.592499 87.707999) (width 0.25) (layer F.Cu) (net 8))
 (segment (start 129.872499 87.207499) (end 126.092999 87.207499) (width 0.25) (layer F.Cu) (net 8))
 (segment (start 130.615 87.95) (end 129.872499 87.207499) (width 0.25) (layer F.Cu) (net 8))
 (segment (start 125.192499 89.532501) (end 124.555 90.17) (width 0.25) (layer F.Cu) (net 8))
 (segment (start 131.315 87.95) (end 130.615 87.95) (width 0.25) (layer F.Cu) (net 8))
 (segment (start 130.615 89.85) (end 131.315 89.85) (width 0.25) (layer F.Cu) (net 7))
 (segment (start 129.972499 89.207499) (end 130.615 89.85) (width 0.25) (layer F.Cu) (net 7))
 (segment (start 127.592499 89.207499) (end 129.972499 89.207499) (width 0.25) (layer F.Cu) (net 7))
 (segment (start 126.555 88.17) (end 127.592499 89.207499) (width 0.25) (layer F.Cu) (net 7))
 (segment (start 132.015 89.85) (end 131.315 89.85) (width 0.25) (layer F.Cu) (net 7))
 (segment (start 132.640001 89.224999) (end 132.015 89.85) (width 0.25) (layer F.Cu) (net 7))
 (segment (start 135.579999 89.224999) (end 132.640001 89.224999) (width 0.25) (layer F.Cu) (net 7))
 (segment (start 140.335 93.98) (end 135.579999 89.224999) (width 0.25) (layer F.Cu) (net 7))
 (segment (start 134.115 89.85) (end 134.115 99.825) (width 0.25) (layer F.Cu) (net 10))
 (segment (start 134.62 100.33) (end 137.795 100.33) (width 0.25) (layer F.Cu) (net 10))
 (segment (start 134.115 99.825) (end 134.62 100.33) (width 0.25) (layer F.Cu) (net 10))
 (segment (start 139.7 100.33) (end 142.24 97.79) (width 0.25) (layer F.Cu) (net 10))
 (segment (start 137.795 100.33) (end 139.7 100.33) (width 0.25) (layer F.Cu) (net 10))
 (segment (start 121.592499 90.10906) (end 121.592499 87.707999) (width 0.25) (layer F.Cu) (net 9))
 (segment (start 121.653439 90.17) (end 121.592499 90.10906) (width 0.25) (layer F.Cu) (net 9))
 (segment (start 122.555 90.17) (end 121.653439 90.17) (width 0.25) (layer F.Cu) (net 9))
 (segment (start 133.415 87.95) (end 134.115 87.95) (width 0.25) (layer F.Cu) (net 9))
 (segment (start 132.22249 86.75749) (end 133.415 87.95) (width 0.25) (layer F.Cu) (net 9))
 (segment (start 122.543008 86.75749) (end 132.22249 86.75749) (width 0.25) (layer F.Cu) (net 9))
 (segment (start 121.592499 87.707999) (end 122.543008 86.75749) (width 0.25) (layer F.Cu) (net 9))
 (segment (start 137.074999 98.510001) (end 136.525 99.06) (width 0.25) (layer B.Cu) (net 9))
 (segment (start 138.820001 96.764999) (end 137.074999 98.510001) (width 0.25) (layer B.Cu) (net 9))
 (segment (start 143.114999 96.764999) (end 138.820001 96.764999) (width 0.25) (layer B.Cu) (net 9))
 (segment (start 144.14 97.79) (end 143.114999 96.764999) (width 0.25) (layer B.Cu) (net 9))
 (segment (start 144.839999 97.090001) (end 144.14 97.79) (width 0.25) (layer F.Cu) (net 9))
 (segment (start 146.490001 95.439999) (end 144.839999 97.090001) (width 0.25) (layer F.Cu) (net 9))
 (segment (start 146.490001 93.463999) (end 146.490001 95.439999) (width 0.25) (layer F.Cu) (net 9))
 (segment (start 140.851001 87.824999) (end 146.490001 93.463999) (width 0.25) (layer F.Cu) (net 9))
 (segment (start 134.940001 87.824999) (end 140.851001 87.824999) (width 0.25) (layer F.Cu) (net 9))
 (segment (start 134.815 87.95) (end 134.940001 87.824999) (width 0.25) (layer F.Cu) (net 9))
 (segment (start 134.115 87.95) (end 134.815 87.95) (width 0.25) (layer F.Cu) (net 9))
 (segment (start 125.517501 89.132501) (end 124.555 88.17) (width 0.25) (layer B.Cu) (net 4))
 (segment (start 125.517501 97.786841) (end 125.517501 89.132501) (width 0.25) (layer B.Cu) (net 4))
 (segment (start 126.365 99.695) (end 126.365 98.63434) (width 0.25) (layer B.Cu) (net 4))
 (segment (start 126.365 98.63434) (end 125.517501 97.786841) (width 0.25) (layer B.Cu) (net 4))
 (segment (start 127.192499 90.807499) (end 126.555 90.17) (width 0.25) (layer F.Cu) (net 3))
 (segment (start 127.517501 91.132501) (end 127.192499 90.807499) (width 0.25) (layer F.Cu) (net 3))
 (segment (start 129.553503 91.132501) (end 127.517501 91.132501) (width 0.25) (layer F.Cu) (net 3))
 (segment (start 132.520001 94.098999) (end 129.553503 91.132501) (width 0.25) (layer F.Cu) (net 3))
 (segment (start 132.520001 98.619999) (end 132.520001 94.098999) (width 0.25) (layer F.Cu) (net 3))
 (segment (start 131.445 99.695) (end 132.520001 98.619999) (width 0.25) (layer F.Cu) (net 3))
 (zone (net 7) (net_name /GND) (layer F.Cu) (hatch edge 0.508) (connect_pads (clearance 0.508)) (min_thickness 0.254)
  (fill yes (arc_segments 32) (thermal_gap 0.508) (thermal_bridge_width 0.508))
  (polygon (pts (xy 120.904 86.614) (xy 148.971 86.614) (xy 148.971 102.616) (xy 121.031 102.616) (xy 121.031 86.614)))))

